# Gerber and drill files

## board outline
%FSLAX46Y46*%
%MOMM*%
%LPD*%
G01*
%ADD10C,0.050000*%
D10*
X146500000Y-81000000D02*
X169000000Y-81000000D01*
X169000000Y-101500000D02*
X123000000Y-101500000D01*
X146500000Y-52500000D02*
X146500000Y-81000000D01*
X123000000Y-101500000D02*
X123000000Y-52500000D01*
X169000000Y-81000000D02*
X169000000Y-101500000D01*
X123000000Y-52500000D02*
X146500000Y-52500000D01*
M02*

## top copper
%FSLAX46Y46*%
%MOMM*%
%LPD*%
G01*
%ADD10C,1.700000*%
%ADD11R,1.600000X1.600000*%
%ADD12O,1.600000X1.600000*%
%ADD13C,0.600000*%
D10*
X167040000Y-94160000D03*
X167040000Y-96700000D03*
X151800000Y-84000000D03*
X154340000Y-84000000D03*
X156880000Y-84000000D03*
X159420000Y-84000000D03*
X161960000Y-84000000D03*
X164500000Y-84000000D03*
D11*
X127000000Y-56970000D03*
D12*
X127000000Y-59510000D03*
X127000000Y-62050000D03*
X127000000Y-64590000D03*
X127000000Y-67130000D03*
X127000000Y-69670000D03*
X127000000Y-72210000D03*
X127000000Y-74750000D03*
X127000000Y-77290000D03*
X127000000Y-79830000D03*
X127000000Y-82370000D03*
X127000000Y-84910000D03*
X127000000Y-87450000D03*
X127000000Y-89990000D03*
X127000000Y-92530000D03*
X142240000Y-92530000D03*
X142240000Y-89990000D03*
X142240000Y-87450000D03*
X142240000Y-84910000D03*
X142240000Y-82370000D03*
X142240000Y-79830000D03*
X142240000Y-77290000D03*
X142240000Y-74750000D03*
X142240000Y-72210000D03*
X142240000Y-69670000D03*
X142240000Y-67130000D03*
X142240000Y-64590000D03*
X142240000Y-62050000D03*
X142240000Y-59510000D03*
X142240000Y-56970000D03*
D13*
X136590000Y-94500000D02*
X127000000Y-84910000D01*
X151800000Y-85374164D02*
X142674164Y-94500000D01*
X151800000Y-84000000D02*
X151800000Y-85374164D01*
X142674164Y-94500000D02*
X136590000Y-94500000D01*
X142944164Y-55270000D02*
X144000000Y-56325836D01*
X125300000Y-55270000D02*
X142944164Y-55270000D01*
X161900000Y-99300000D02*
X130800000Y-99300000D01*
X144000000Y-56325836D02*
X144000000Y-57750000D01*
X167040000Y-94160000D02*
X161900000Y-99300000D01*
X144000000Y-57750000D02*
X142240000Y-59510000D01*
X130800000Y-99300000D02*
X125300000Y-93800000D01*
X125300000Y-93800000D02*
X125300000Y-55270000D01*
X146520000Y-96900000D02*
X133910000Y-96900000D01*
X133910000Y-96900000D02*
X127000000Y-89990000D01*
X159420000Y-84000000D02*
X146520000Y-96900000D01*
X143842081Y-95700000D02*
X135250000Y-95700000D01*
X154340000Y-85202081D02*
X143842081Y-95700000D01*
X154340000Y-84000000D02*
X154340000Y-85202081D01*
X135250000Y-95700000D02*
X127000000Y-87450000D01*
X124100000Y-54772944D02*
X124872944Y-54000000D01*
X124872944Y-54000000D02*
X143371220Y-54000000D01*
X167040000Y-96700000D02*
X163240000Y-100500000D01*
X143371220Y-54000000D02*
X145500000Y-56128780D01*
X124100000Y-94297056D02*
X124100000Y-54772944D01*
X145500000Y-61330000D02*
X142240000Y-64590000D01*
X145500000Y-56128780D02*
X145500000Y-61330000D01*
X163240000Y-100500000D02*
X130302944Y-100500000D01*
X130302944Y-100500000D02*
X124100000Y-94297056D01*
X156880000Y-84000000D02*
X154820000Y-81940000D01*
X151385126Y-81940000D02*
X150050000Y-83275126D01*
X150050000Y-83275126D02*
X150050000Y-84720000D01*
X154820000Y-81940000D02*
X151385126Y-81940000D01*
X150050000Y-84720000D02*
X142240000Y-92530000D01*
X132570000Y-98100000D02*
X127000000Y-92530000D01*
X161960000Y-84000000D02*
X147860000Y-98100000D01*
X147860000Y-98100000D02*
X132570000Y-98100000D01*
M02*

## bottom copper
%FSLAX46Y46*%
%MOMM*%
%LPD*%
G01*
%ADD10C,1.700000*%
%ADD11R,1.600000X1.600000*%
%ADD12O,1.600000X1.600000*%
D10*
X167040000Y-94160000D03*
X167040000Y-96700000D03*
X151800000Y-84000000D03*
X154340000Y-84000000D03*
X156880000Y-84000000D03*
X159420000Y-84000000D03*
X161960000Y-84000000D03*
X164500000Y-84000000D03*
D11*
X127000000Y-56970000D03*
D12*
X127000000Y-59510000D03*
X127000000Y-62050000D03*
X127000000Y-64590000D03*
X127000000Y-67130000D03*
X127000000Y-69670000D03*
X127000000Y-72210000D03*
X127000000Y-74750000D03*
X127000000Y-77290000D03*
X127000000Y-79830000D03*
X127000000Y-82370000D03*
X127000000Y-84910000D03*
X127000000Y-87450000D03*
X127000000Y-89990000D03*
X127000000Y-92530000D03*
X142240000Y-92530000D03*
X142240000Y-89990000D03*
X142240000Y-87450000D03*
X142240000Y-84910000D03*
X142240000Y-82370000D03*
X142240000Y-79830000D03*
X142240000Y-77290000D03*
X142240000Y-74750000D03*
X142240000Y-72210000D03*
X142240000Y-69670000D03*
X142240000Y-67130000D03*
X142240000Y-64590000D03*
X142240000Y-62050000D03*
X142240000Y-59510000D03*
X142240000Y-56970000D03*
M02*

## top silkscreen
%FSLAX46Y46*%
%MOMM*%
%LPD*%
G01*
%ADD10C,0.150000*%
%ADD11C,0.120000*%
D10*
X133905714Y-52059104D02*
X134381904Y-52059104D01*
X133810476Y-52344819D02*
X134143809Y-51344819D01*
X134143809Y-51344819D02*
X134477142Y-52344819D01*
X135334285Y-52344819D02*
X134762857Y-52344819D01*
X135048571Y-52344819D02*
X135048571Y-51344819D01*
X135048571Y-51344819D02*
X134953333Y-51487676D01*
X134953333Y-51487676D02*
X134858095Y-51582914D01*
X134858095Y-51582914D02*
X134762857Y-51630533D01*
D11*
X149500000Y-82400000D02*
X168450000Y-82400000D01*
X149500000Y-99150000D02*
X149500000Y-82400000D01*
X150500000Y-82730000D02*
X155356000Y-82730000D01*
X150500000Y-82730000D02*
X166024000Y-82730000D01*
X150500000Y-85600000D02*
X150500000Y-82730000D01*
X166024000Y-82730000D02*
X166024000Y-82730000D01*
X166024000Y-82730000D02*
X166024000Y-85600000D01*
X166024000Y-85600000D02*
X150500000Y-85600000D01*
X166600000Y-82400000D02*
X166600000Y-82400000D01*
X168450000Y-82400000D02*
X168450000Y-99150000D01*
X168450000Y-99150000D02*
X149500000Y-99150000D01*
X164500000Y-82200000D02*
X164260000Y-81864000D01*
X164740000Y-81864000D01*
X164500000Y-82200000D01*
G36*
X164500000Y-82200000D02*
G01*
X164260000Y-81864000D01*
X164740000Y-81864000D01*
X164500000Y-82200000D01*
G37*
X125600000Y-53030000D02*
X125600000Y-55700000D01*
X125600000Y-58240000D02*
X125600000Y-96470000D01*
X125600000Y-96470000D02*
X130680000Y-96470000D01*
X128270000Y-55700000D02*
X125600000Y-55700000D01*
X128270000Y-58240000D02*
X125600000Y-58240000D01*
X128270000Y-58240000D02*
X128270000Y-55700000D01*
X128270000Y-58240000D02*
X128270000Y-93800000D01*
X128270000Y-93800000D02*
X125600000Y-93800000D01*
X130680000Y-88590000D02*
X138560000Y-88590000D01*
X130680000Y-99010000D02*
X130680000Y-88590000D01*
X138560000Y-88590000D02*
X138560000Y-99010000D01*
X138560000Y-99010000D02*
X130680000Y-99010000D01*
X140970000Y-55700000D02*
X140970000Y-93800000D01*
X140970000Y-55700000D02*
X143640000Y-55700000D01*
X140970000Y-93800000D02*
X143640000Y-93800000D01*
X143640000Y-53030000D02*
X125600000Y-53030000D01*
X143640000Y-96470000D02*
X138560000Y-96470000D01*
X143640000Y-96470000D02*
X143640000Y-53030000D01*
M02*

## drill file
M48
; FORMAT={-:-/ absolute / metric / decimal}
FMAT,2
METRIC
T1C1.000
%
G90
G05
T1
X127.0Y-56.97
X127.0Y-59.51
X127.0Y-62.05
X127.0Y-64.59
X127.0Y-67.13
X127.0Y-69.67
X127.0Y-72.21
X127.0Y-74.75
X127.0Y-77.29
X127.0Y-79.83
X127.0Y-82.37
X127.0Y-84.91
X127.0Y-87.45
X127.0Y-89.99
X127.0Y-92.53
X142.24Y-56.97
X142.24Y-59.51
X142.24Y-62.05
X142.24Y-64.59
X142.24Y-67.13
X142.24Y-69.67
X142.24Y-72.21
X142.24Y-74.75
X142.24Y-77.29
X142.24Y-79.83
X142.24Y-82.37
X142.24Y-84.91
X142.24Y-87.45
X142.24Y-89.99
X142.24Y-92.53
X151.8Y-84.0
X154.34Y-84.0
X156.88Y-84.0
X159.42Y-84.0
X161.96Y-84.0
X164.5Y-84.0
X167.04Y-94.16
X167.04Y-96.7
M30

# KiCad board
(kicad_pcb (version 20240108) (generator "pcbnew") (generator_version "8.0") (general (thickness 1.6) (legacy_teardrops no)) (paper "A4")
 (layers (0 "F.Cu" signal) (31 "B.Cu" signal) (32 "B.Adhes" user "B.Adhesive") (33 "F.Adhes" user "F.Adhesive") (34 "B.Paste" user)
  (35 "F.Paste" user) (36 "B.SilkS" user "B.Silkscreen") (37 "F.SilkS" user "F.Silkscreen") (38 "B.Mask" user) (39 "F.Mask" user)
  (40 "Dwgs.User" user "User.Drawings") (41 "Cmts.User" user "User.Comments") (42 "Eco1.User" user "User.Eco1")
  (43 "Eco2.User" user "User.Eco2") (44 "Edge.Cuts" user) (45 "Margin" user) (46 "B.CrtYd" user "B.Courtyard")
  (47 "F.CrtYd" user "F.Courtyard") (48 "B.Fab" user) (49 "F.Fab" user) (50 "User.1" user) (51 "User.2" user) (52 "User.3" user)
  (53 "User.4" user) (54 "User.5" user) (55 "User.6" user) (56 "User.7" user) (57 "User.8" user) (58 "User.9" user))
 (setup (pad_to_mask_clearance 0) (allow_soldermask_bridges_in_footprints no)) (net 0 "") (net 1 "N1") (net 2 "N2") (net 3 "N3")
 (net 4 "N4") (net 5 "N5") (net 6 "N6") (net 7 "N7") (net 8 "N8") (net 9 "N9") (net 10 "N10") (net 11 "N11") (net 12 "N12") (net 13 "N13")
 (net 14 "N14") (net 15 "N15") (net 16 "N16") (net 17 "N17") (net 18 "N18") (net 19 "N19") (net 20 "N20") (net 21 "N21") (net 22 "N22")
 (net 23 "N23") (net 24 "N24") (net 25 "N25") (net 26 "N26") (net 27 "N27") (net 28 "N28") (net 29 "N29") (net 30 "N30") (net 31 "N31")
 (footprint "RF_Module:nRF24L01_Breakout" (layer "F.Cu") (at 164.5 84 -90)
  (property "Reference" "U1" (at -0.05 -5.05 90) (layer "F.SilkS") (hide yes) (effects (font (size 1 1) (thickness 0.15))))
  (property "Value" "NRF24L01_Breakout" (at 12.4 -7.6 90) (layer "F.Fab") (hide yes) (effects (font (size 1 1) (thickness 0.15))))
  (fp_line (start -1.6 15) (end -1.6 -3.95) (stroke (width 0.12) (type solid)) (layer "F.SilkS"))
  (fp_line (start 15.15 15) (end -1.6 15) (stroke (width 0.12) (type solid)) (layer "F.SilkS"))
  (fp_line (start -1.27 14) (end -1.27 9.144) (stroke (width 0.12) (type solid)) (layer "F.SilkS"))
  (fp_line (start -1.27 14) (end -1.27 -1.524) (stroke (width 0.12) (type solid)) (layer "F.SilkS"))
  (fp_line (start 1.6 14) (end -1.27 14) (stroke (width 0.12) (type solid)) (layer "F.SilkS"))
  (fp_line (start -1.27 -1.524) (end -1.27 -1.524) (stroke (width 0.12) (type solid)) (layer "F.SilkS"))
  (fp_line (start -1.27 -1.524) (end 1.6 -1.524) (stroke (width 0.12) (type solid)) (layer "F.SilkS"))
  (fp_line (start 1.6 -1.524) (end 1.6 14) (stroke (width 0.12) (type solid)) (layer "F.SilkS"))
  (fp_line (start -1.6 -2.1) (end -1.6 -2.1) (stroke (width 0.12) (type solid)) (layer "F.SilkS"))
  (fp_line (start -1.6 -3.95) (end 15.15 -3.95) (stroke (width 0.12) (type solid)) (layer "F.SilkS"))
  (fp_line (start 15.15 -3.95) (end 15.15 15) (stroke (width 0.12) (type solid)) (layer "F.SilkS"))
  (fp_poly
   (pts (xy -1.8 0) (xy -2.136 0.24) (xy -2.136 -0.24) (xy -1.8 0)) (stroke (width 0.12) (type solid)) (fill solid) (layer "F.SilkS"))
  (pad "1" thru_hole circle (at 10.16 -2.54 270) (size 1.7 1.7) (drill 1) (layers "*.Cu" "*.Mask") (remove_unused_layers no) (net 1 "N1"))
  (pad "2" thru_hole circle (at 12.7 -2.54 270) (size 1.7 1.7) (drill 1) (layers "*.Cu" "*.Mask") (remove_unused_layers no) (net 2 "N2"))
  (pad "3" thru_hole circle (at 0 12.7 270) (size 1.7 1.7) (drill 1) (layers "*.Cu" "*.Mask") (remove_unused_layers no) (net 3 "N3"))
  (pad "4" thru_hole circle (at 0 10.16 270) (size 1.7 1.7) (drill 1) (layers "*.Cu" "*.Mask") (remove_unused_layers no) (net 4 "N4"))
  (pad "5" thru_hole circle (at 0 7.62 270) (size 1.7 1.7) (drill 1) (layers "*.Cu" "*.Mask") (remove_unused_layers no) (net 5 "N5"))
  (pad "6" thru_hole circle (at 0 5.08 270) (size 1.7 1.7) (drill 1) (layers "*.Cu" "*.Mask") (remove_unused_layers no) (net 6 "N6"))
  (pad "7" thru_hole circle (at 0 2.54 270) (size 1.7 1.7) (drill 1) (layers "*.Cu" "*.Mask") (remove_unused_layers no) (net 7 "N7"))
  (pad "8" thru_hole circle (at 0 0 270) (size 1.7 1.7) (drill 1) (layers "*.Cu" "*.Mask") (remove_unused_layers no) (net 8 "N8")))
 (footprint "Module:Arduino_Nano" (layer "F.Cu") (at 127 56.97)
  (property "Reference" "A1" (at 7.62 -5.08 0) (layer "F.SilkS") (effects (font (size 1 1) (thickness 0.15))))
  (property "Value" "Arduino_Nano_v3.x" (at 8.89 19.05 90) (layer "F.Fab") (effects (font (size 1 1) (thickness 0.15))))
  (fp_line (start -1.4 -3.94) (end -1.4 -1.27) (stroke (width 0.12) (type solid)) (layer "F.SilkS"))
  (fp_line (start -1.4 1.27) (end -1.4 39.5) (stroke (width 0.12) (type solid)) (layer "F.SilkS"))
  (fp_line (start -1.4 39.5) (end 3.68 39.5) (stroke (width 0.12) (type solid)) (layer "F.SilkS"))
  (fp_line (start 1.27 -1.27) (end -1.4 -1.27) (stroke (width 0.12) (type solid)) (layer "F.SilkS"))
  (fp_line (start 1.27 1.27) (end -1.4 1.27) (stroke (width 0.12) (type solid)) (layer "F.SilkS"))
  (fp_line (start 1.27 1.27) (end 1.27 -1.27) (stroke (width 0.12) (type solid)) (layer "F.SilkS"))
  (fp_line (start 1.27 1.27) (end 1.27 36.83) (stroke (width 0.12) (type solid)) (layer "F.SilkS"))
  (fp_line (start 1.27 36.83) (end -1.4 36.83) (stroke (width 0.12) (type solid)) (layer "F.SilkS"))
  (fp_line (start 3.68 31.62) (end 11.56 31.62) (stroke (width 0.12) (type solid)) (layer "F.SilkS"))
  (fp_line (start 3.68 42.04) (end 3.68 31.62) (stroke (width 0.12) (type solid)) (layer "F.SilkS"))
  (fp_line (start 11.56 31.62) (end 11.56 42.04) (stroke (width 0.12) (type solid)) (layer "F.SilkS"))
  (fp_line (start 11.56 42.04) (end 3.68 42.04) (stroke (width 0.12) (type solid)) (layer "F.SilkS"))
  (fp_line (start 13.97 -1.27) (end 13.97 36.83) (stroke (width 0.12) (type solid)) (layer "F.SilkS"))
  (fp_line (start 13.97 -1.27) (end 16.64 -1.27) (stroke (width 0.12) (type solid)) (layer "F.SilkS"))
  (fp_line (start 13.97 36.83) (end 16.64 36.83) (stroke (width 0.12) (type solid)) (layer "F.SilkS"))
  (fp_line (start 16.64 -3.94) (end -1.4 -3.94) (stroke (width 0.12) (type solid)) (layer "F.SilkS"))
  (fp_line (start 16.64 39.5) (end 11.56 39.5) (stroke (width 0.12) (type solid)) (layer "F.SilkS"))
  (fp_line (start 16.64 39.5) (end 16.64 -3.94) (stroke (width 0.12) (type solid)) (layer "F.SilkS"))
  (pad "1" thru_hole rect (at 0 0) (size 1.6 1.6) (drill 1) (layers "*.Cu" "*.Mask") (remove_unused_layers no) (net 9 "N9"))
  (pad "2" thru_hole oval (at 0 2.54) (size 1.6 1.6) (drill 1) (layers "*.Cu" "*.Mask") (remove_unused_layers no) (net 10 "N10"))
  (pad "3" thru_hole oval (at 0 5.08) (size 1.6 1.6) (drill 1) (layers "*.Cu" "*.Mask") (remove_unused_layers no) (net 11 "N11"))
  (pad "4" thru_hole oval (at 0 7.62) (size 1.6 1.6) (drill 1) (layers "*.Cu" "*.Mask") (remove_unused_layers no) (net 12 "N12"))
  (pad "5" thru_hole oval (at 0 10.16) (size 1.6 1.6) (drill 1) (layers "*.Cu" "*.Mask") (remove_unused_layers no) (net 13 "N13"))
  (pad "6" thru_hole oval (at 0 12.7) (size 1.6 1.6) (drill 1) (layers "*.Cu" "*.Mask") (remove_unused_layers no) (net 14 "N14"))
  (pad "7" thru_hole oval (at 0 15.24) (size 1.6 1.6) (drill 1) (layers "*.Cu" "*.Mask") (remove_unused_layers no) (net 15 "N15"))
  (pad "8" thru_hole oval (at 0 17.78) (size 1.6 1.6) (drill 1) (layers "*.Cu" "*.Mask") (remove_unused_layers no) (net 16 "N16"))
  (pad "9" thru_hole oval (at 0 20.32) (size 1.6 1.6) (drill 1) (layers "*.Cu" "*.Mask") (remove_unused_layers no) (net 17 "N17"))
  (pad "10" thru_hole oval (at 0 22.86) (size 1.6 1.6) (drill 1) (layers "*.Cu" "*.Mask") (remove_unused_layers no) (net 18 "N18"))
  (pad "11" thru_hole oval (at 0 25.4) (size 1.6 1.6) (drill 1) (layers "*.Cu" "*.Mask") (remove_unused_layers no) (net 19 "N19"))
  (pad "12" thru_hole oval (at 0 27.94) (size 1.6 1.6) (drill 1) (layers "*.Cu" "*.Mask") (remove_unused_layers no) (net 3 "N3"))
  (pad "13" thru_hole oval (at 0 30.48) (size 1.6 1.6) (drill 1) (layers "*.Cu" "*.Mask") (remove_unused_layers no) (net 4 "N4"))
  (pad "14" thru_hole oval (at 0 33.02) (size 1.6 1.6) (drill 1) (layers "*.Cu" "*.Mask") (remove_unused_layers no) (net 6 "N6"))
  (pad "15" thru_hole oval (at 0 35.56) (size 1.6 1.6) (drill 1) (layers "*.Cu" "*.Mask") (remove_unused_layers no) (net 7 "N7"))
  (pad "16" thru_hole oval (at 15.24 35.56) (size 1.6 1.6) (drill 1) (layers "*.Cu" "*.Mask") (remove_unused_layers no) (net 5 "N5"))
  (pad "17" thru_hole oval (at 15.24 33.02) (size 1.6 1.6) (drill 1) (layers "*.Cu" "*.Mask") (remove_unused_layers no) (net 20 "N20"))
  (pad "18" thru_hole oval (at 15.24 30.48) (size 1.6 1.6) (drill 1) (layers "*.Cu" "*.Mask") (remove_unused_layers no) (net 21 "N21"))
  (pad "19" thru_hole oval (at 15.24 27.94) (size 1.6 1.6) (drill 1) (layers "*.Cu" "*.Mask") (remove_unused_layers no) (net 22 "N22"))
  (pad "20" thru_hole oval (at 15.24 25.4) (size 1.6 1.6) (drill 1) (layers "*.Cu" "*.Mask") (remove_unused_layers no) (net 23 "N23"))
  (pad "21" thru_hole oval (at 15.24 22.86) (size 1.6 1.6) (drill 1) (layers "*.Cu" "*.Mask") (remove_unused_layers no) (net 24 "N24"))
  (pad "22" thru_hole oval (at 15.24 20.32) (size 1.6 1.6) (drill 1) (layers "*.Cu" "*.Mask") (remove_unused_layers no) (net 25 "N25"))
  (pad "23" thru_hole oval (at 15.24 17.78) (size 1.6 1.6) (drill 1) (layers "*.Cu" "*.Mask") (remove_unused_layers no) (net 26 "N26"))
  (pad "24" thru_hole oval (at 15.24 15.24) (size 1.6 1.6) (drill 1) (layers "*.Cu" "*.Mask") (remove_unused_layers no) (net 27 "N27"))
  (pad "25" thru_hole oval (at 15.24 12.7) (size 1.6 1.6) (drill 1) (layers "*.Cu" "*.Mask") (remove_unused_layers no) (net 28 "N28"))
  (pad "26" thru_hole oval (at 15.24 10.16) (size 1.6 1.6) (drill 1) (layers "*.Cu" "*.Mask") (remove_unused_layers no) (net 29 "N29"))
  (pad "27" thru_hole oval (at 15.24 7.62) (size 1.6 1.6) (drill 1) (layers "*.Cu" "*.Mask") (remove_unused_layers no) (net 2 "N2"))
  (pad "28" thru_hole oval (at 15.24 5.08) (size 1.6 1.6) (drill 1) (layers "*.Cu" "*.Mask") (remove_unused_layers no) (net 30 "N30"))
  (pad "29" thru_hole oval (at 15.24 2.54) (size 1.6 1.6) (drill 1) (layers "*.Cu" "*.Mask") (remove_unused_layers no) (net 1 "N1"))
  (pad "30" thru_hole oval (at 15.24 0) (size 1.6 1.6) (drill 1) (layers "*.Cu" "*.Mask") (remove_unused_layers no) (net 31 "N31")))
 (gr_line (start 146.5 81) (end 169 81) (stroke (width 0.05) (type default)) (layer "Edge.Cuts"))
 (gr_line (start 169 101.5) (end 123 101.5) (stroke (width 0.05) (type default)) (layer "Edge.Cuts"))
 (gr_line (start 146.5 52.5) (end 146.5 81) (stroke (width 0.05) (type default)) (layer "Edge.Cuts"))
 (gr_line (start 123 101.5) (end 123 52.5) (stroke (width 0.05) (type default)) (layer "Edge.Cuts"))
 (gr_line (start 169 81) (end 169 101.5) (stroke (width 0.05) (type default)) (layer "Edge.Cuts"))
 (gr_line (start 123 52.5) (end 146.5 52.5) (stroke (width 0.05) (type default)) (layer "Edge.Cuts"))
 (segment (start 136.59 94.5) (end 127 84.91) (width 0.6) (layer "F.Cu") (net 3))
 (segment (start 151.8 85.374164) (end 142.674164 94.5) (width 0.6) (layer "F.Cu") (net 3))
 (segment (start 151.8 84) (end 151.8 85.374164) (width 0.6) (layer "F.Cu") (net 3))
 (segment (start 142.674164 94.5) (end 136.59 94.5) (width 0.6) (layer "F.Cu") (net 3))
 (segment (start 142.944164 55.27) (end 144 56.325836) (width 0.6) (layer "F.Cu") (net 1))
 (segment (start 125.3 55.27) (end 142.944164 55.27) (width 0.6) (layer "F.Cu") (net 1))
 (segment (start 161.9 99.3) (end 130.8 99.3) (width 0.6) (layer "F.Cu") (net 1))
 (segment (start 144 56.325836) (end 144 57.75) (width 0.6) (layer "F.Cu") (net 1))
 (segment (start 167.04 94.16) (end 161.9 99.3) (width 0.6) (layer "F.Cu") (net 1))
 (segment (start 144 57.75) (end 142.24 59.51) (width 0.6) (layer "F.Cu") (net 1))
 (segment (start 130.8 99.3) (end 125.3 93.8) (width 0.6) (layer "F.Cu") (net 1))
 (segment (start 125.3 93.8) (end 125.3 55.27) (width 0.6) (layer "F.Cu") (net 1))
 (segment (start 146.52 96.9) (end 133.91 96.9) (width 0.6) (layer "F.Cu") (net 6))
 (segment (start 133.91 96.9) (end 127 89.99) (width 0.6) (layer "F.Cu") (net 6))
 (segment (start 159.42 84) (end 146.52 96.9) (width 0.6) (layer "F.Cu") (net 6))
 (segment (start 143.842081 95.7) (end 135.25 95.7) (width 0.6) (layer "F.Cu") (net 4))
 (segment (start 154.34 85.202081) (end 143.842081 95.7) (width 0.6) (layer "F.Cu") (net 4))
 (segment (start 154.34 84) (end 154.34 85.202081) (width 0.6) (layer "F.Cu") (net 4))
 (segment (start 135.25 95.7) (end 127 87.45) (width 0.6) (layer "F.Cu") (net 4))
 (segment (start 124.1 54.772944) (end 124.872944 54) (width 0.6) (layer "F.Cu") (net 2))
 (segment (start 124.872944 54) (end 143.37122 54) (width 0.6) (layer "F.Cu") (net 2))
 (segment (start 167.04 96.7) (end 163.24 100.5) (width 0.6) (layer "F.Cu") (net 2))
 (segment (start 143.37122 54) (end 145.5 56.12878) (width 0.6) (layer "F.Cu") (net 2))
 (segment (start 124.1 94.297056) (end 124.1 54.772944) (width 0.6) (layer "F.Cu") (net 2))
 (segment (start 145.5 61.33) (end 142.24 64.59) (width 0.6) (layer "F.Cu") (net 2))
 (segment (start 145.5 56.12878) (end 145.5 61.33) (width 0.6) (layer "F.Cu") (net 2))
 (segment (start 163.24 100.5) (end 130.302944 100.5) (width 0.6) (layer "F.Cu") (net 2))
 (segment (start 130.302944 100.5) (end 124.1 94.297056) (width 0.6) (layer "F.Cu") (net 2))
 (segment (start 156.88 84) (end 154.82 81.94) (width 0.6) (layer "F.Cu") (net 5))
 (segment (start 151.385126 81.94) (end 150.05 83.275126) (width 0.6) (layer "F.Cu") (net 5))
 (segment (start 150.05 83.275126) (end 150.05 84.72) (width 0.6) (layer "F.Cu") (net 5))
 (segment (start 154.82 81.94) (end 151.385126 81.94) (width 0.6) (layer "F.Cu") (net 5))
 (segment (start 150.05 84.72) (end 142.24 92.53) (width 0.6) (layer "F.Cu") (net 5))
 (segment (start 132.57 98.1) (end 127 92.53) (width 0.6) (layer "F.Cu") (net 7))
 (segment (start 161.96 84) (end 147.86 98.1) (width 0.6) (layer "F.Cu") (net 7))
 (segment (start 147.86 98.1) (end 132.57 98.1) (width 0.6) (layer "F.Cu") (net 7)))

